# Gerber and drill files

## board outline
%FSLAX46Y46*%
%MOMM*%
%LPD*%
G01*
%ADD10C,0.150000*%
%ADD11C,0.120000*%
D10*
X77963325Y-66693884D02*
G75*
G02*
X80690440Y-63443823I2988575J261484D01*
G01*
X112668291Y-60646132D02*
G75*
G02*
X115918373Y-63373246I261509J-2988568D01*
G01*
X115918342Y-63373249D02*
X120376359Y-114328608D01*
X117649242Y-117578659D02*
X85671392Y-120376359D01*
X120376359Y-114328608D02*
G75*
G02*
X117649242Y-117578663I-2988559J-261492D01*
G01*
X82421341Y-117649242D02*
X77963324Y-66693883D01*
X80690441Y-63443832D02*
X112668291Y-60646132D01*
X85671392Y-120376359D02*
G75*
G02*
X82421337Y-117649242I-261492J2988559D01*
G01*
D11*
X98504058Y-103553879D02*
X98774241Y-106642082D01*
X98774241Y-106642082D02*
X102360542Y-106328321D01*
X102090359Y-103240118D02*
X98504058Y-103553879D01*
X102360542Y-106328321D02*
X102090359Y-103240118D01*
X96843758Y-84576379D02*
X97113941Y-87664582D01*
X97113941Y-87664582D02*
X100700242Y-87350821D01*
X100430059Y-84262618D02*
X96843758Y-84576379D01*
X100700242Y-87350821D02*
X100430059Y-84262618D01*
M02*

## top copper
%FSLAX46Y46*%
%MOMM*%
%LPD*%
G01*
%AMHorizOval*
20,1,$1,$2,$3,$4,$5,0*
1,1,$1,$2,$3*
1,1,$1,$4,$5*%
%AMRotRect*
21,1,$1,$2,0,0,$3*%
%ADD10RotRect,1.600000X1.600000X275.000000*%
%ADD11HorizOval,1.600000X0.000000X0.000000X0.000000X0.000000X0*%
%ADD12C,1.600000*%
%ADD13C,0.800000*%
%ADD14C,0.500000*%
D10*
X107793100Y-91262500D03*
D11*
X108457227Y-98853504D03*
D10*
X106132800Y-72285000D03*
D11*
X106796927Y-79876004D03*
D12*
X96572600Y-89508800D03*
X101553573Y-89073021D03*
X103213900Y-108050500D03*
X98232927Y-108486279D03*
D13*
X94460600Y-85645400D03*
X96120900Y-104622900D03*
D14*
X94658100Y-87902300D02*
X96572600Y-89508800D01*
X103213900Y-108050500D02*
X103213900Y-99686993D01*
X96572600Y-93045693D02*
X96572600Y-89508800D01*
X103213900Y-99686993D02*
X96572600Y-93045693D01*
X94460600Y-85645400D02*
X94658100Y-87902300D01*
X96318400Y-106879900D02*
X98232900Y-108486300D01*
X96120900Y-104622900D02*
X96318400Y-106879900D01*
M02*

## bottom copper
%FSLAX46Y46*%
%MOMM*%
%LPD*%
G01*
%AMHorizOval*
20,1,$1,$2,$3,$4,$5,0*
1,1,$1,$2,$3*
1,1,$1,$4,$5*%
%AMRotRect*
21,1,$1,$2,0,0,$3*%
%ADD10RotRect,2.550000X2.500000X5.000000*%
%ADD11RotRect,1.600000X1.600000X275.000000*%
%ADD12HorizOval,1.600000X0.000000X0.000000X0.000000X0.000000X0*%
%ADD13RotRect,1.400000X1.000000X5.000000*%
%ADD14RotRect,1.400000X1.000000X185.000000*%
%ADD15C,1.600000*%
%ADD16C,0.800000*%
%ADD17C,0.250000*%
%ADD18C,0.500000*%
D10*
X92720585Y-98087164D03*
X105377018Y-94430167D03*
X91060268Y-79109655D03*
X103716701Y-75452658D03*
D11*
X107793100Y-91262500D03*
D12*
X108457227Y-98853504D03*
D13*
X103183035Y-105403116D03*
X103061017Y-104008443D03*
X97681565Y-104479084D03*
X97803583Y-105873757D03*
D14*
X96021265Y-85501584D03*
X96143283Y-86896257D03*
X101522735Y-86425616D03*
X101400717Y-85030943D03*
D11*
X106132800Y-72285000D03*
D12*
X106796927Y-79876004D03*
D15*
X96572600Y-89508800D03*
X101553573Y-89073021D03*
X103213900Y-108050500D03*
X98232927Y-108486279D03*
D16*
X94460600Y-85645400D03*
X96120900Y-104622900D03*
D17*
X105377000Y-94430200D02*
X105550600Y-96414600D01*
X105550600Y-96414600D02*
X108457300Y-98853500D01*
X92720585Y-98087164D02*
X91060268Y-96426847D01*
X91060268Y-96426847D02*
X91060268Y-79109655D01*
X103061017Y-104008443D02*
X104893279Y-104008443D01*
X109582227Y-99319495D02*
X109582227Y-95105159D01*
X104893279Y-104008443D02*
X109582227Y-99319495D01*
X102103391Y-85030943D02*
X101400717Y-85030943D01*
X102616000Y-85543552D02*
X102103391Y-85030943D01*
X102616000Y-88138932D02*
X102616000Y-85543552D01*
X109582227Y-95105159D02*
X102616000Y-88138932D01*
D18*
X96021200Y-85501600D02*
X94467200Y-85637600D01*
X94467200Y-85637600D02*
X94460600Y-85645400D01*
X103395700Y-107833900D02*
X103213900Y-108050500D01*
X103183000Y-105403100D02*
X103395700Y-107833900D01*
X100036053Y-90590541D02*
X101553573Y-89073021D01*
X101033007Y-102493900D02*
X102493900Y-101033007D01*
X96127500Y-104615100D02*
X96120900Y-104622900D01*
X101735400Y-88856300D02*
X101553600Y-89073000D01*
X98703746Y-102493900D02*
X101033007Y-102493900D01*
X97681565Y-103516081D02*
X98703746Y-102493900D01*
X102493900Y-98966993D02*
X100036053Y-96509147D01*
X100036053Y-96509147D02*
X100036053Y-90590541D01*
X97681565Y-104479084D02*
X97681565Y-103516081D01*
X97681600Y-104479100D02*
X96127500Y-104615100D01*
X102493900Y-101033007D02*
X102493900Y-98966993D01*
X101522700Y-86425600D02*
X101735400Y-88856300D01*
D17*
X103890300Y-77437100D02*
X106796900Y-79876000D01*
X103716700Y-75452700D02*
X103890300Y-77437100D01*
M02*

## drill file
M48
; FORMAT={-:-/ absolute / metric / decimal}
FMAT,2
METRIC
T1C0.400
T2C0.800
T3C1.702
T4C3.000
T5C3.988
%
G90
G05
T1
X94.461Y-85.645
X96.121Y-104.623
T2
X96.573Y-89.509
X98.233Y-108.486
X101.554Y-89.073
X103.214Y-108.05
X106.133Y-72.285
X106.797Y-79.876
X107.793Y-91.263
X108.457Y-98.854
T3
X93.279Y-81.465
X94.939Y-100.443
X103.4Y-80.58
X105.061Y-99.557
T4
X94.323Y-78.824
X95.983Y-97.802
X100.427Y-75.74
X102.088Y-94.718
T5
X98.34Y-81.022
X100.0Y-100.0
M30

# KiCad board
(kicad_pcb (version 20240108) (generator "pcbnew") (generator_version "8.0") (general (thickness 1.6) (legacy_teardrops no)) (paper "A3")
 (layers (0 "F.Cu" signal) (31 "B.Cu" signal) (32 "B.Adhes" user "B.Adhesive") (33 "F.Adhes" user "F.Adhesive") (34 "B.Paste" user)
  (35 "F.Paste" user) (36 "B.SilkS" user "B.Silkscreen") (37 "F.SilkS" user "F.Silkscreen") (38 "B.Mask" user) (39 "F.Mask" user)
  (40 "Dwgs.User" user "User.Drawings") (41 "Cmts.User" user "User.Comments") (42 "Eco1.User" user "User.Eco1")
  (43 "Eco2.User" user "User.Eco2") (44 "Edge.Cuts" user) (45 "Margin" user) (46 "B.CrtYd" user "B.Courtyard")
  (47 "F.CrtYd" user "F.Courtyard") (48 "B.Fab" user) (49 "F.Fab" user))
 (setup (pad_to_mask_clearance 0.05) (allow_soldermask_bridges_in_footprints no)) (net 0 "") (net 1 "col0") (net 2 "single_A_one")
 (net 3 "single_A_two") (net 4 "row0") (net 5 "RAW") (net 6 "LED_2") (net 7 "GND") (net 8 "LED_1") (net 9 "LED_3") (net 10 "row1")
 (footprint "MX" (layer "F.Cu") (at 100 100 5)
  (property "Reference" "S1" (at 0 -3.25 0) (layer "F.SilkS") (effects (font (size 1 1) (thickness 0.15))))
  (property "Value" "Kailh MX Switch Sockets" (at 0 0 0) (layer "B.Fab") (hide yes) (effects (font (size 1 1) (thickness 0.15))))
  (pad "" np_thru_hole circle (at -5.08 0) (size 1.7018 1.7018) (drill 1.7018) (layers "*.Cu" "*.Mask"))
  (pad "" np_thru_hole circle (at -3.81 -2.54) (size 3 3) (drill 3) (layers "*.Cu" "*.Mask"))
  (pad "" np_thru_hole circle (at 0 0) (size 3.9878 3.9878) (drill 3.9878) (layers "*.Cu" "*.Mask"))
  (pad "" np_thru_hole circle (at 2.54 -5.08) (size 3 3) (drill 3) (layers "*.Cu" "*.Mask"))
  (pad "" np_thru_hole circle (at 5.08 0) (size 1.7018 1.7018) (drill 1.7018) (layers "*.Cu" "*.Mask"))
  (pad "1" smd rect (at -7.085 -2.54 5) (size 2.55 2.5) (layers "B.Cu" "B.Paste" "B.Mask") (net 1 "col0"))
  (pad "2" smd rect (at 5.842 -5.08 5) (size 2.55 2.5) (layers "B.Cu" "B.Paste" "B.Mask") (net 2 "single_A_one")))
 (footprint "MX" (layer "F.Cu") (at 98.339683 81.022491 5)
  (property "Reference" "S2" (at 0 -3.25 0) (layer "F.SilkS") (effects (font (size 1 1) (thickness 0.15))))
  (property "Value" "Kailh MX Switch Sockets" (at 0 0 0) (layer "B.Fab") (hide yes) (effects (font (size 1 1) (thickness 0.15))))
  (pad "" np_thru_hole circle (at -5.08 0) (size 1.7018 1.7018) (drill 1.7018) (layers "*.Cu" "*.Mask"))
  (pad "" np_thru_hole circle (at -3.81 -2.54) (size 3 3) (drill 3) (layers "*.Cu" "*.Mask"))
  (pad "" np_thru_hole circle (at 0 0) (size 3.9878 3.9878) (drill 3.9878) (layers "*.Cu" "*.Mask"))
  (pad "" np_thru_hole circle (at 2.54 -5.08) (size 3 3) (drill 3) (layers "*.Cu" "*.Mask"))
  (pad "" np_thru_hole circle (at 5.08 0) (size 1.7018 1.7018) (drill 1.7018) (layers "*.Cu" "*.Mask"))
  (pad "1" smd rect (at -7.085 -2.54 5) (size 2.55 2.5) (layers "B.Cu" "B.Paste" "B.Mask") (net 1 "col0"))
  (pad "2" smd rect (at 5.842 -5.08 5) (size 2.55 2.5) (layers "B.Cu" "B.Paste" "B.Mask") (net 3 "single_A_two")))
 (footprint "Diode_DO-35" (layer "B.Cu") (at 107.7931 91.2625 -85)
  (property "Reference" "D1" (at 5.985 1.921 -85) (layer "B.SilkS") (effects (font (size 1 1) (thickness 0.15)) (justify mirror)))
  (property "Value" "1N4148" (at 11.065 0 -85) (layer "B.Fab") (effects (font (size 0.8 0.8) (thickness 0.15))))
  (pad "1" thru_hole rect (at 0 0 275) (size 1.6 1.6) (drill 0.8) (layers "*.Cu" "*.Mask") (remove_unused_layers no) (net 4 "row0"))
  (pad "2" thru_hole oval (at 7.62 0 275) (size 1.6 1.6) (drill 0.8) (layers "*.Cu" "*.Mask") (remove_unused_layers no)
   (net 2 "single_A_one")))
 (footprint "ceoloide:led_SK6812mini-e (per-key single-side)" (layer "B.Cu") (at 100.4323 104.9411 5)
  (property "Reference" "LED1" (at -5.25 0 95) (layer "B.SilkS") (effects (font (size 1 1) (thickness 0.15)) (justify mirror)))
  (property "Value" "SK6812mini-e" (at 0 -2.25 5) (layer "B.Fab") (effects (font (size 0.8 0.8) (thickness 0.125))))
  (fp_line (start -1.8 -1.55) (end -1.8 1.55) (stroke (width 0.12) (type solid)) (layer "Edge.Cuts"))
  (fp_line (start -1.8 1.55) (end 1.8 1.55) (stroke (width 0.12) (type solid)) (layer "Edge.Cuts"))
  (fp_line (start 1.8 -1.55) (end -1.8 -1.55) (stroke (width 0.12) (type solid)) (layer "Edge.Cuts"))
  (fp_line (start 1.8 1.55) (end 1.8 -1.55) (stroke (width 0.12) (type solid)) (layer "Edge.Cuts"))
  (pad "1" smd rect (at 2.7 0.7 5) (size 1.4 1) (layers "B.Cu" "B.Paste" "B.Mask") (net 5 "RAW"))
  (pad "2" smd rect (at 2.7 -0.7 5) (size 1.4 1) (layers "B.Cu" "B.Paste" "B.Mask") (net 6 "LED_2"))
  (pad "3" smd rect (at -2.7 -0.7 5) (size 1.4 1) (layers "B.Cu" "B.Paste" "B.Mask") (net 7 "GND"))
  (pad "4" smd rect (at -2.7 0.7 5) (size 1.4 1) (layers "B.Cu" "B.Paste" "B.Mask") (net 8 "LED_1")))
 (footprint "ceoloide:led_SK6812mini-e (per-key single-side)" (layer "B.Cu") (at 98.772 85.9636 -175)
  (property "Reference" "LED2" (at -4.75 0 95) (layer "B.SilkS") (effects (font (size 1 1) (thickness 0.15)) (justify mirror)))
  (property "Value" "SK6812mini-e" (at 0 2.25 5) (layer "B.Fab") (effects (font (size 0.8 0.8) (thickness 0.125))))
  (fp_line (start 1.8 1.55) (end 1.8 -1.55) (stroke (width 0.12) (type solid)) (layer "Edge.Cuts"))
  (fp_line (start 1.8 -1.55) (end -1.8 -1.55) (stroke (width 0.12) (type solid)) (layer "Edge.Cuts"))
  (fp_line (start -1.8 1.55) (end 1.8 1.55) (stroke (width 0.12) (type solid)) (layer "Edge.Cuts"))
  (fp_line (start -1.8 -1.55) (end -1.8 1.55) (stroke (width 0.12) (type solid)) (layer "Edge.Cuts"))
  (pad "1" smd rect (at 2.7 0.7 185) (size 1.4 1) (layers "B.Cu" "B.Paste" "B.Mask") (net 5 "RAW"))
  (pad "2" smd rect (at 2.7 -0.7 185) (size 1.4 1) (layers "B.Cu" "B.Paste" "B.Mask") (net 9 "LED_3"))
  (pad "3" smd rect (at -2.7 -0.7 185) (size 1.4 1) (layers "B.Cu" "B.Paste" "B.Mask") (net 7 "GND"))
  (pad "4" smd rect (at -2.7 0.7 185) (size 1.4 1) (layers "B.Cu" "B.Paste" "B.Mask") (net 6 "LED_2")))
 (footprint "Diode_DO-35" (layer "B.Cu") (at 106.1328 72.285 -85)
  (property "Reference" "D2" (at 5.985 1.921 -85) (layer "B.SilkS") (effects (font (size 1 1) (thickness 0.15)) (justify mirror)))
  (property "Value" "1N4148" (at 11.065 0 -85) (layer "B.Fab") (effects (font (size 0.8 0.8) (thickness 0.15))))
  (pad "1" thru_hole rect (at 0 0 275) (size 1.6 1.6) (drill 0.8) (layers "*.Cu" "*.Mask") (remove_unused_layers no) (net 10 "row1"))
  (pad "2" thru_hole oval (at 7.62 0 275) (size 1.6 1.6) (drill 0.8) (layers "*.Cu" "*.Mask") (remove_unused_layers no)
   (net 3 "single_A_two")))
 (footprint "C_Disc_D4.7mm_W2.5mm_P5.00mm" (layer "B.Cu") (at 96.5726 89.5088 5)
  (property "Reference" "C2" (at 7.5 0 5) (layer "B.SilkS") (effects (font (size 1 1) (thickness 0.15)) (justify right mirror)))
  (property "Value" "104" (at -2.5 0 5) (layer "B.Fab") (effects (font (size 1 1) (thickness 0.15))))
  (pad "1" thru_hole circle (at 0 0) (size 1.6 1.6) (drill 0.8) (layers "*.Cu" "*.Mask") (remove_unused_layers no) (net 5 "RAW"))
  (pad "2" thru_hole circle (at 5 0) (size 1.6 1.6) (drill 0.8) (layers "*.Cu" "*.Mask") (remove_unused_layers no) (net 7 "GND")))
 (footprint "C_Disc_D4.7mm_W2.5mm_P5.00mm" (layer "B.Cu") (at 103.2139 108.0505 -175)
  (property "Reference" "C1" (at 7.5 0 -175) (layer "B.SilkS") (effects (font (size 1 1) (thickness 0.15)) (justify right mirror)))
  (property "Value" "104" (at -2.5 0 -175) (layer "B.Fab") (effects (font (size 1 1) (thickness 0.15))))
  (pad "1" thru_hole circle (at 0 0) (size 1.6 1.6) (drill 0.8) (layers "*.Cu" "*.Mask") (remove_unused_layers no) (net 5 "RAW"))
  (pad "2" thru_hole circle (at 5 0) (size 1.6 1.6) (drill 0.8) (layers "*.Cu" "*.Mask") (remove_unused_layers no) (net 7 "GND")))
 (gr_arc (start 77.963325 66.693884) (mid 78.653775 64.504054) (end 80.690441 63.443832) (stroke (width 0.15) (type solid))
  (layer "Edge.Cuts"))
 (gr_arc (start 112.668291 60.646132) (mid 114.858121 61.336583) (end 115.918342 63.373249) (stroke (width 0.15) (type solid))
  (layer "Edge.Cuts"))
 (gr_line (start 115.918342 63.373249) (end 120.376359 114.328608) (stroke (width 0.15) (type solid)) (layer "Edge.Cuts"))
 (gr_line (start 117.649242 117.578659) (end 85.671392 120.376359) (stroke (width 0.15) (type solid)) (layer "Edge.Cuts"))
 (gr_arc (start 120.376359 114.328608) (mid 119.685908 116.518438) (end 117.649242 117.578659) (stroke (width 0.15) (type solid))
  (layer "Edge.Cuts"))
 (gr_line (start 82.421341 117.649242) (end 77.963324 66.693883) (stroke (width 0.15) (type solid)) (layer "Edge.Cuts"))
 (gr_line (start 80.690441 63.443832) (end 112.668291 60.646132) (stroke (width 0.15) (type solid)) (layer "Edge.Cuts"))
 (gr_arc (start 85.671392 120.376359) (mid 83.481562 119.685908) (end 82.421341 117.649242) (stroke (width 0.15) (type solid))
  (layer "Edge.Cuts"))
 (segment (start 105.377 94.4302) (end 105.5506 96.4146) (width 0.25) (layer "B.Cu") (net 2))
 (segment (start 105.5506 96.4146) (end 108.4573 98.8535) (width 0.25) (layer "B.Cu") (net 2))
 (segment (start 92.720585 98.087164) (end 91.060268 96.426847) (width 0.25) (layer "B.Cu") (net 1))
 (segment (start 91.060268 96.426847) (end 91.060268 79.109655) (width 0.25) (layer "B.Cu") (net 1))
 (segment (start 103.061017 104.008443) (end 104.893279 104.008443) (width 0.25) (layer "B.Cu") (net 6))
 (segment (start 109.582227 99.319495) (end 109.582227 95.105159) (width 0.25) (layer "B.Cu") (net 6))
 (segment (start 104.893279 104.008443) (end 109.582227 99.319495) (width 0.25) (layer "B.Cu") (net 6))
 (segment (start 102.103391 85.030943) (end 101.400717 85.030943) (width 0.25) (layer "B.Cu") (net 6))
 (segment (start 102.616 85.543552) (end 102.103391 85.030943) (width 0.25) (layer "B.Cu") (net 6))
 (segment (start 102.616 88.138932) (end 102.616 85.543552) (width 0.25) (layer "B.Cu") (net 6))
 (segment (start 109.582227 95.105159) (end 102.616 88.138932) (width 0.25) (layer "B.Cu") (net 6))
 (segment (start 94.6581 87.9023) (end 96.5726 89.5088) (width 0.5) (layer "F.Cu") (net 5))
 (segment (start 103.2139 108.0505) (end 103.2139 99.686993) (width 0.5) (layer "F.Cu") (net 5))
 (segment (start 96.5726 93.045693) (end 96.5726 89.5088) (width 0.5) (layer "F.Cu") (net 5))
 (segment (start 103.2139 99.686993) (end 96.5726 93.045693) (width 0.5) (layer "F.Cu") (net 5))
 (segment (start 94.4606 85.6454) (end 94.6581 87.9023) (width 0.5) (layer "F.Cu") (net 5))
 (via (at 94.4606 85.6454) (size 0.8) (drill 0.4) (layers "F.Cu" "B.Cu") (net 5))
 (segment (start 96.0212 85.5016) (end 94.4672 85.6376) (width 0.5) (layer "B.Cu") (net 5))
 (segment (start 94.4672 85.6376) (end 94.4606 85.6454) (width 0.5) (layer "B.Cu") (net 5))
 (segment (start 103.3957 107.8339) (end 103.2139 108.0505) (width 0.5) (layer "B.Cu") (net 5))
 (segment (start 103.183 105.4031) (end 103.3957 107.8339) (width 0.5) (layer "B.Cu") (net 5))
 (segment (start 96.3184 106.8799) (end 98.2329 108.4863) (width 0.5) (layer "F.Cu") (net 7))
 (segment (start 96.1209 104.6229) (end 96.3184 106.8799) (width 0.5) (layer "F.Cu") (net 7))
 (via (at 96.1209 104.6229) (size 0.8) (drill 0.4) (layers "F.Cu" "B.Cu") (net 7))
 (segment (start 100.036053 90.590541) (end 101.553573 89.073021) (width 0.5) (layer "B.Cu") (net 7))
 (segment (start 101.033007 102.4939) (end 102.4939 101.033007) (width 0.5) (layer "B.Cu") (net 7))
 (segment (start 96.1275 104.6151) (end 96.1209 104.6229) (width 0.5) (layer "B.Cu") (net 7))
 (segment (start 101.7354 88.8563) (end 101.5536 89.073) (width 0.5) (layer "B.Cu") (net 7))
 (segment (start 98.703746 102.4939) (end 101.033007 102.4939) (width 0.5) (layer "B.Cu") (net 7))
 (segment (start 97.681565 103.516081) (end 98.703746 102.4939) (width 0.5) (layer "B.Cu") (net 7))
 (segment (start 102.4939 98.966993) (end 100.036053 96.509147) (width 0.5) (layer "B.Cu") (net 7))
 (segment (start 100.036053 96.509147) (end 100.036053 90.590541) (width 0.5) (layer "B.Cu") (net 7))
 (segment (start 97.681565 104.479084) (end 97.681565 103.516081) (width 0.5) (layer "B.Cu") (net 7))
 (segment (start 97.6816 104.4791) (end 96.1275 104.6151) (width 0.5) (layer "B.Cu") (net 7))
 (segment (start 102.4939 101.033007) (end 102.4939 98.966993) (width 0.5) (layer "B.Cu") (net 7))
 (segment (start 101.5227 86.4256) (end 101.7354 88.8563) (width 0.5) (layer "B.Cu") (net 7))
 (segment (start 103.8903 77.4371) (end 106.7969 79.876) (width 0.25) (layer "B.Cu") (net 3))
 (segment (start 103.7167 75.4527) (end 103.8903 77.4371) (width 0.25) (layer "B.Cu") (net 3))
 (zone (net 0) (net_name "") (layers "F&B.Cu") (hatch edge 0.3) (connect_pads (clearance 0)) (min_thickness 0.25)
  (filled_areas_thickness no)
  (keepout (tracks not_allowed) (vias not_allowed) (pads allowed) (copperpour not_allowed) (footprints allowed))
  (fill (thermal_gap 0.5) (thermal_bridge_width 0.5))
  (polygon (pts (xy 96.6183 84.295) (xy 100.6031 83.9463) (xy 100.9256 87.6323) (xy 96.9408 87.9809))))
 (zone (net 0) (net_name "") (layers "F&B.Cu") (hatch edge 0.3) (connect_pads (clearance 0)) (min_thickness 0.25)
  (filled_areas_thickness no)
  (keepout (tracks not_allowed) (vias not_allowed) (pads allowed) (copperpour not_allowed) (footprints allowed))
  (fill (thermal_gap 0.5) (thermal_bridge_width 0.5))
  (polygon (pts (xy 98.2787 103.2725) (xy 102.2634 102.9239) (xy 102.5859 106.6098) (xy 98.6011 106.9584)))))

